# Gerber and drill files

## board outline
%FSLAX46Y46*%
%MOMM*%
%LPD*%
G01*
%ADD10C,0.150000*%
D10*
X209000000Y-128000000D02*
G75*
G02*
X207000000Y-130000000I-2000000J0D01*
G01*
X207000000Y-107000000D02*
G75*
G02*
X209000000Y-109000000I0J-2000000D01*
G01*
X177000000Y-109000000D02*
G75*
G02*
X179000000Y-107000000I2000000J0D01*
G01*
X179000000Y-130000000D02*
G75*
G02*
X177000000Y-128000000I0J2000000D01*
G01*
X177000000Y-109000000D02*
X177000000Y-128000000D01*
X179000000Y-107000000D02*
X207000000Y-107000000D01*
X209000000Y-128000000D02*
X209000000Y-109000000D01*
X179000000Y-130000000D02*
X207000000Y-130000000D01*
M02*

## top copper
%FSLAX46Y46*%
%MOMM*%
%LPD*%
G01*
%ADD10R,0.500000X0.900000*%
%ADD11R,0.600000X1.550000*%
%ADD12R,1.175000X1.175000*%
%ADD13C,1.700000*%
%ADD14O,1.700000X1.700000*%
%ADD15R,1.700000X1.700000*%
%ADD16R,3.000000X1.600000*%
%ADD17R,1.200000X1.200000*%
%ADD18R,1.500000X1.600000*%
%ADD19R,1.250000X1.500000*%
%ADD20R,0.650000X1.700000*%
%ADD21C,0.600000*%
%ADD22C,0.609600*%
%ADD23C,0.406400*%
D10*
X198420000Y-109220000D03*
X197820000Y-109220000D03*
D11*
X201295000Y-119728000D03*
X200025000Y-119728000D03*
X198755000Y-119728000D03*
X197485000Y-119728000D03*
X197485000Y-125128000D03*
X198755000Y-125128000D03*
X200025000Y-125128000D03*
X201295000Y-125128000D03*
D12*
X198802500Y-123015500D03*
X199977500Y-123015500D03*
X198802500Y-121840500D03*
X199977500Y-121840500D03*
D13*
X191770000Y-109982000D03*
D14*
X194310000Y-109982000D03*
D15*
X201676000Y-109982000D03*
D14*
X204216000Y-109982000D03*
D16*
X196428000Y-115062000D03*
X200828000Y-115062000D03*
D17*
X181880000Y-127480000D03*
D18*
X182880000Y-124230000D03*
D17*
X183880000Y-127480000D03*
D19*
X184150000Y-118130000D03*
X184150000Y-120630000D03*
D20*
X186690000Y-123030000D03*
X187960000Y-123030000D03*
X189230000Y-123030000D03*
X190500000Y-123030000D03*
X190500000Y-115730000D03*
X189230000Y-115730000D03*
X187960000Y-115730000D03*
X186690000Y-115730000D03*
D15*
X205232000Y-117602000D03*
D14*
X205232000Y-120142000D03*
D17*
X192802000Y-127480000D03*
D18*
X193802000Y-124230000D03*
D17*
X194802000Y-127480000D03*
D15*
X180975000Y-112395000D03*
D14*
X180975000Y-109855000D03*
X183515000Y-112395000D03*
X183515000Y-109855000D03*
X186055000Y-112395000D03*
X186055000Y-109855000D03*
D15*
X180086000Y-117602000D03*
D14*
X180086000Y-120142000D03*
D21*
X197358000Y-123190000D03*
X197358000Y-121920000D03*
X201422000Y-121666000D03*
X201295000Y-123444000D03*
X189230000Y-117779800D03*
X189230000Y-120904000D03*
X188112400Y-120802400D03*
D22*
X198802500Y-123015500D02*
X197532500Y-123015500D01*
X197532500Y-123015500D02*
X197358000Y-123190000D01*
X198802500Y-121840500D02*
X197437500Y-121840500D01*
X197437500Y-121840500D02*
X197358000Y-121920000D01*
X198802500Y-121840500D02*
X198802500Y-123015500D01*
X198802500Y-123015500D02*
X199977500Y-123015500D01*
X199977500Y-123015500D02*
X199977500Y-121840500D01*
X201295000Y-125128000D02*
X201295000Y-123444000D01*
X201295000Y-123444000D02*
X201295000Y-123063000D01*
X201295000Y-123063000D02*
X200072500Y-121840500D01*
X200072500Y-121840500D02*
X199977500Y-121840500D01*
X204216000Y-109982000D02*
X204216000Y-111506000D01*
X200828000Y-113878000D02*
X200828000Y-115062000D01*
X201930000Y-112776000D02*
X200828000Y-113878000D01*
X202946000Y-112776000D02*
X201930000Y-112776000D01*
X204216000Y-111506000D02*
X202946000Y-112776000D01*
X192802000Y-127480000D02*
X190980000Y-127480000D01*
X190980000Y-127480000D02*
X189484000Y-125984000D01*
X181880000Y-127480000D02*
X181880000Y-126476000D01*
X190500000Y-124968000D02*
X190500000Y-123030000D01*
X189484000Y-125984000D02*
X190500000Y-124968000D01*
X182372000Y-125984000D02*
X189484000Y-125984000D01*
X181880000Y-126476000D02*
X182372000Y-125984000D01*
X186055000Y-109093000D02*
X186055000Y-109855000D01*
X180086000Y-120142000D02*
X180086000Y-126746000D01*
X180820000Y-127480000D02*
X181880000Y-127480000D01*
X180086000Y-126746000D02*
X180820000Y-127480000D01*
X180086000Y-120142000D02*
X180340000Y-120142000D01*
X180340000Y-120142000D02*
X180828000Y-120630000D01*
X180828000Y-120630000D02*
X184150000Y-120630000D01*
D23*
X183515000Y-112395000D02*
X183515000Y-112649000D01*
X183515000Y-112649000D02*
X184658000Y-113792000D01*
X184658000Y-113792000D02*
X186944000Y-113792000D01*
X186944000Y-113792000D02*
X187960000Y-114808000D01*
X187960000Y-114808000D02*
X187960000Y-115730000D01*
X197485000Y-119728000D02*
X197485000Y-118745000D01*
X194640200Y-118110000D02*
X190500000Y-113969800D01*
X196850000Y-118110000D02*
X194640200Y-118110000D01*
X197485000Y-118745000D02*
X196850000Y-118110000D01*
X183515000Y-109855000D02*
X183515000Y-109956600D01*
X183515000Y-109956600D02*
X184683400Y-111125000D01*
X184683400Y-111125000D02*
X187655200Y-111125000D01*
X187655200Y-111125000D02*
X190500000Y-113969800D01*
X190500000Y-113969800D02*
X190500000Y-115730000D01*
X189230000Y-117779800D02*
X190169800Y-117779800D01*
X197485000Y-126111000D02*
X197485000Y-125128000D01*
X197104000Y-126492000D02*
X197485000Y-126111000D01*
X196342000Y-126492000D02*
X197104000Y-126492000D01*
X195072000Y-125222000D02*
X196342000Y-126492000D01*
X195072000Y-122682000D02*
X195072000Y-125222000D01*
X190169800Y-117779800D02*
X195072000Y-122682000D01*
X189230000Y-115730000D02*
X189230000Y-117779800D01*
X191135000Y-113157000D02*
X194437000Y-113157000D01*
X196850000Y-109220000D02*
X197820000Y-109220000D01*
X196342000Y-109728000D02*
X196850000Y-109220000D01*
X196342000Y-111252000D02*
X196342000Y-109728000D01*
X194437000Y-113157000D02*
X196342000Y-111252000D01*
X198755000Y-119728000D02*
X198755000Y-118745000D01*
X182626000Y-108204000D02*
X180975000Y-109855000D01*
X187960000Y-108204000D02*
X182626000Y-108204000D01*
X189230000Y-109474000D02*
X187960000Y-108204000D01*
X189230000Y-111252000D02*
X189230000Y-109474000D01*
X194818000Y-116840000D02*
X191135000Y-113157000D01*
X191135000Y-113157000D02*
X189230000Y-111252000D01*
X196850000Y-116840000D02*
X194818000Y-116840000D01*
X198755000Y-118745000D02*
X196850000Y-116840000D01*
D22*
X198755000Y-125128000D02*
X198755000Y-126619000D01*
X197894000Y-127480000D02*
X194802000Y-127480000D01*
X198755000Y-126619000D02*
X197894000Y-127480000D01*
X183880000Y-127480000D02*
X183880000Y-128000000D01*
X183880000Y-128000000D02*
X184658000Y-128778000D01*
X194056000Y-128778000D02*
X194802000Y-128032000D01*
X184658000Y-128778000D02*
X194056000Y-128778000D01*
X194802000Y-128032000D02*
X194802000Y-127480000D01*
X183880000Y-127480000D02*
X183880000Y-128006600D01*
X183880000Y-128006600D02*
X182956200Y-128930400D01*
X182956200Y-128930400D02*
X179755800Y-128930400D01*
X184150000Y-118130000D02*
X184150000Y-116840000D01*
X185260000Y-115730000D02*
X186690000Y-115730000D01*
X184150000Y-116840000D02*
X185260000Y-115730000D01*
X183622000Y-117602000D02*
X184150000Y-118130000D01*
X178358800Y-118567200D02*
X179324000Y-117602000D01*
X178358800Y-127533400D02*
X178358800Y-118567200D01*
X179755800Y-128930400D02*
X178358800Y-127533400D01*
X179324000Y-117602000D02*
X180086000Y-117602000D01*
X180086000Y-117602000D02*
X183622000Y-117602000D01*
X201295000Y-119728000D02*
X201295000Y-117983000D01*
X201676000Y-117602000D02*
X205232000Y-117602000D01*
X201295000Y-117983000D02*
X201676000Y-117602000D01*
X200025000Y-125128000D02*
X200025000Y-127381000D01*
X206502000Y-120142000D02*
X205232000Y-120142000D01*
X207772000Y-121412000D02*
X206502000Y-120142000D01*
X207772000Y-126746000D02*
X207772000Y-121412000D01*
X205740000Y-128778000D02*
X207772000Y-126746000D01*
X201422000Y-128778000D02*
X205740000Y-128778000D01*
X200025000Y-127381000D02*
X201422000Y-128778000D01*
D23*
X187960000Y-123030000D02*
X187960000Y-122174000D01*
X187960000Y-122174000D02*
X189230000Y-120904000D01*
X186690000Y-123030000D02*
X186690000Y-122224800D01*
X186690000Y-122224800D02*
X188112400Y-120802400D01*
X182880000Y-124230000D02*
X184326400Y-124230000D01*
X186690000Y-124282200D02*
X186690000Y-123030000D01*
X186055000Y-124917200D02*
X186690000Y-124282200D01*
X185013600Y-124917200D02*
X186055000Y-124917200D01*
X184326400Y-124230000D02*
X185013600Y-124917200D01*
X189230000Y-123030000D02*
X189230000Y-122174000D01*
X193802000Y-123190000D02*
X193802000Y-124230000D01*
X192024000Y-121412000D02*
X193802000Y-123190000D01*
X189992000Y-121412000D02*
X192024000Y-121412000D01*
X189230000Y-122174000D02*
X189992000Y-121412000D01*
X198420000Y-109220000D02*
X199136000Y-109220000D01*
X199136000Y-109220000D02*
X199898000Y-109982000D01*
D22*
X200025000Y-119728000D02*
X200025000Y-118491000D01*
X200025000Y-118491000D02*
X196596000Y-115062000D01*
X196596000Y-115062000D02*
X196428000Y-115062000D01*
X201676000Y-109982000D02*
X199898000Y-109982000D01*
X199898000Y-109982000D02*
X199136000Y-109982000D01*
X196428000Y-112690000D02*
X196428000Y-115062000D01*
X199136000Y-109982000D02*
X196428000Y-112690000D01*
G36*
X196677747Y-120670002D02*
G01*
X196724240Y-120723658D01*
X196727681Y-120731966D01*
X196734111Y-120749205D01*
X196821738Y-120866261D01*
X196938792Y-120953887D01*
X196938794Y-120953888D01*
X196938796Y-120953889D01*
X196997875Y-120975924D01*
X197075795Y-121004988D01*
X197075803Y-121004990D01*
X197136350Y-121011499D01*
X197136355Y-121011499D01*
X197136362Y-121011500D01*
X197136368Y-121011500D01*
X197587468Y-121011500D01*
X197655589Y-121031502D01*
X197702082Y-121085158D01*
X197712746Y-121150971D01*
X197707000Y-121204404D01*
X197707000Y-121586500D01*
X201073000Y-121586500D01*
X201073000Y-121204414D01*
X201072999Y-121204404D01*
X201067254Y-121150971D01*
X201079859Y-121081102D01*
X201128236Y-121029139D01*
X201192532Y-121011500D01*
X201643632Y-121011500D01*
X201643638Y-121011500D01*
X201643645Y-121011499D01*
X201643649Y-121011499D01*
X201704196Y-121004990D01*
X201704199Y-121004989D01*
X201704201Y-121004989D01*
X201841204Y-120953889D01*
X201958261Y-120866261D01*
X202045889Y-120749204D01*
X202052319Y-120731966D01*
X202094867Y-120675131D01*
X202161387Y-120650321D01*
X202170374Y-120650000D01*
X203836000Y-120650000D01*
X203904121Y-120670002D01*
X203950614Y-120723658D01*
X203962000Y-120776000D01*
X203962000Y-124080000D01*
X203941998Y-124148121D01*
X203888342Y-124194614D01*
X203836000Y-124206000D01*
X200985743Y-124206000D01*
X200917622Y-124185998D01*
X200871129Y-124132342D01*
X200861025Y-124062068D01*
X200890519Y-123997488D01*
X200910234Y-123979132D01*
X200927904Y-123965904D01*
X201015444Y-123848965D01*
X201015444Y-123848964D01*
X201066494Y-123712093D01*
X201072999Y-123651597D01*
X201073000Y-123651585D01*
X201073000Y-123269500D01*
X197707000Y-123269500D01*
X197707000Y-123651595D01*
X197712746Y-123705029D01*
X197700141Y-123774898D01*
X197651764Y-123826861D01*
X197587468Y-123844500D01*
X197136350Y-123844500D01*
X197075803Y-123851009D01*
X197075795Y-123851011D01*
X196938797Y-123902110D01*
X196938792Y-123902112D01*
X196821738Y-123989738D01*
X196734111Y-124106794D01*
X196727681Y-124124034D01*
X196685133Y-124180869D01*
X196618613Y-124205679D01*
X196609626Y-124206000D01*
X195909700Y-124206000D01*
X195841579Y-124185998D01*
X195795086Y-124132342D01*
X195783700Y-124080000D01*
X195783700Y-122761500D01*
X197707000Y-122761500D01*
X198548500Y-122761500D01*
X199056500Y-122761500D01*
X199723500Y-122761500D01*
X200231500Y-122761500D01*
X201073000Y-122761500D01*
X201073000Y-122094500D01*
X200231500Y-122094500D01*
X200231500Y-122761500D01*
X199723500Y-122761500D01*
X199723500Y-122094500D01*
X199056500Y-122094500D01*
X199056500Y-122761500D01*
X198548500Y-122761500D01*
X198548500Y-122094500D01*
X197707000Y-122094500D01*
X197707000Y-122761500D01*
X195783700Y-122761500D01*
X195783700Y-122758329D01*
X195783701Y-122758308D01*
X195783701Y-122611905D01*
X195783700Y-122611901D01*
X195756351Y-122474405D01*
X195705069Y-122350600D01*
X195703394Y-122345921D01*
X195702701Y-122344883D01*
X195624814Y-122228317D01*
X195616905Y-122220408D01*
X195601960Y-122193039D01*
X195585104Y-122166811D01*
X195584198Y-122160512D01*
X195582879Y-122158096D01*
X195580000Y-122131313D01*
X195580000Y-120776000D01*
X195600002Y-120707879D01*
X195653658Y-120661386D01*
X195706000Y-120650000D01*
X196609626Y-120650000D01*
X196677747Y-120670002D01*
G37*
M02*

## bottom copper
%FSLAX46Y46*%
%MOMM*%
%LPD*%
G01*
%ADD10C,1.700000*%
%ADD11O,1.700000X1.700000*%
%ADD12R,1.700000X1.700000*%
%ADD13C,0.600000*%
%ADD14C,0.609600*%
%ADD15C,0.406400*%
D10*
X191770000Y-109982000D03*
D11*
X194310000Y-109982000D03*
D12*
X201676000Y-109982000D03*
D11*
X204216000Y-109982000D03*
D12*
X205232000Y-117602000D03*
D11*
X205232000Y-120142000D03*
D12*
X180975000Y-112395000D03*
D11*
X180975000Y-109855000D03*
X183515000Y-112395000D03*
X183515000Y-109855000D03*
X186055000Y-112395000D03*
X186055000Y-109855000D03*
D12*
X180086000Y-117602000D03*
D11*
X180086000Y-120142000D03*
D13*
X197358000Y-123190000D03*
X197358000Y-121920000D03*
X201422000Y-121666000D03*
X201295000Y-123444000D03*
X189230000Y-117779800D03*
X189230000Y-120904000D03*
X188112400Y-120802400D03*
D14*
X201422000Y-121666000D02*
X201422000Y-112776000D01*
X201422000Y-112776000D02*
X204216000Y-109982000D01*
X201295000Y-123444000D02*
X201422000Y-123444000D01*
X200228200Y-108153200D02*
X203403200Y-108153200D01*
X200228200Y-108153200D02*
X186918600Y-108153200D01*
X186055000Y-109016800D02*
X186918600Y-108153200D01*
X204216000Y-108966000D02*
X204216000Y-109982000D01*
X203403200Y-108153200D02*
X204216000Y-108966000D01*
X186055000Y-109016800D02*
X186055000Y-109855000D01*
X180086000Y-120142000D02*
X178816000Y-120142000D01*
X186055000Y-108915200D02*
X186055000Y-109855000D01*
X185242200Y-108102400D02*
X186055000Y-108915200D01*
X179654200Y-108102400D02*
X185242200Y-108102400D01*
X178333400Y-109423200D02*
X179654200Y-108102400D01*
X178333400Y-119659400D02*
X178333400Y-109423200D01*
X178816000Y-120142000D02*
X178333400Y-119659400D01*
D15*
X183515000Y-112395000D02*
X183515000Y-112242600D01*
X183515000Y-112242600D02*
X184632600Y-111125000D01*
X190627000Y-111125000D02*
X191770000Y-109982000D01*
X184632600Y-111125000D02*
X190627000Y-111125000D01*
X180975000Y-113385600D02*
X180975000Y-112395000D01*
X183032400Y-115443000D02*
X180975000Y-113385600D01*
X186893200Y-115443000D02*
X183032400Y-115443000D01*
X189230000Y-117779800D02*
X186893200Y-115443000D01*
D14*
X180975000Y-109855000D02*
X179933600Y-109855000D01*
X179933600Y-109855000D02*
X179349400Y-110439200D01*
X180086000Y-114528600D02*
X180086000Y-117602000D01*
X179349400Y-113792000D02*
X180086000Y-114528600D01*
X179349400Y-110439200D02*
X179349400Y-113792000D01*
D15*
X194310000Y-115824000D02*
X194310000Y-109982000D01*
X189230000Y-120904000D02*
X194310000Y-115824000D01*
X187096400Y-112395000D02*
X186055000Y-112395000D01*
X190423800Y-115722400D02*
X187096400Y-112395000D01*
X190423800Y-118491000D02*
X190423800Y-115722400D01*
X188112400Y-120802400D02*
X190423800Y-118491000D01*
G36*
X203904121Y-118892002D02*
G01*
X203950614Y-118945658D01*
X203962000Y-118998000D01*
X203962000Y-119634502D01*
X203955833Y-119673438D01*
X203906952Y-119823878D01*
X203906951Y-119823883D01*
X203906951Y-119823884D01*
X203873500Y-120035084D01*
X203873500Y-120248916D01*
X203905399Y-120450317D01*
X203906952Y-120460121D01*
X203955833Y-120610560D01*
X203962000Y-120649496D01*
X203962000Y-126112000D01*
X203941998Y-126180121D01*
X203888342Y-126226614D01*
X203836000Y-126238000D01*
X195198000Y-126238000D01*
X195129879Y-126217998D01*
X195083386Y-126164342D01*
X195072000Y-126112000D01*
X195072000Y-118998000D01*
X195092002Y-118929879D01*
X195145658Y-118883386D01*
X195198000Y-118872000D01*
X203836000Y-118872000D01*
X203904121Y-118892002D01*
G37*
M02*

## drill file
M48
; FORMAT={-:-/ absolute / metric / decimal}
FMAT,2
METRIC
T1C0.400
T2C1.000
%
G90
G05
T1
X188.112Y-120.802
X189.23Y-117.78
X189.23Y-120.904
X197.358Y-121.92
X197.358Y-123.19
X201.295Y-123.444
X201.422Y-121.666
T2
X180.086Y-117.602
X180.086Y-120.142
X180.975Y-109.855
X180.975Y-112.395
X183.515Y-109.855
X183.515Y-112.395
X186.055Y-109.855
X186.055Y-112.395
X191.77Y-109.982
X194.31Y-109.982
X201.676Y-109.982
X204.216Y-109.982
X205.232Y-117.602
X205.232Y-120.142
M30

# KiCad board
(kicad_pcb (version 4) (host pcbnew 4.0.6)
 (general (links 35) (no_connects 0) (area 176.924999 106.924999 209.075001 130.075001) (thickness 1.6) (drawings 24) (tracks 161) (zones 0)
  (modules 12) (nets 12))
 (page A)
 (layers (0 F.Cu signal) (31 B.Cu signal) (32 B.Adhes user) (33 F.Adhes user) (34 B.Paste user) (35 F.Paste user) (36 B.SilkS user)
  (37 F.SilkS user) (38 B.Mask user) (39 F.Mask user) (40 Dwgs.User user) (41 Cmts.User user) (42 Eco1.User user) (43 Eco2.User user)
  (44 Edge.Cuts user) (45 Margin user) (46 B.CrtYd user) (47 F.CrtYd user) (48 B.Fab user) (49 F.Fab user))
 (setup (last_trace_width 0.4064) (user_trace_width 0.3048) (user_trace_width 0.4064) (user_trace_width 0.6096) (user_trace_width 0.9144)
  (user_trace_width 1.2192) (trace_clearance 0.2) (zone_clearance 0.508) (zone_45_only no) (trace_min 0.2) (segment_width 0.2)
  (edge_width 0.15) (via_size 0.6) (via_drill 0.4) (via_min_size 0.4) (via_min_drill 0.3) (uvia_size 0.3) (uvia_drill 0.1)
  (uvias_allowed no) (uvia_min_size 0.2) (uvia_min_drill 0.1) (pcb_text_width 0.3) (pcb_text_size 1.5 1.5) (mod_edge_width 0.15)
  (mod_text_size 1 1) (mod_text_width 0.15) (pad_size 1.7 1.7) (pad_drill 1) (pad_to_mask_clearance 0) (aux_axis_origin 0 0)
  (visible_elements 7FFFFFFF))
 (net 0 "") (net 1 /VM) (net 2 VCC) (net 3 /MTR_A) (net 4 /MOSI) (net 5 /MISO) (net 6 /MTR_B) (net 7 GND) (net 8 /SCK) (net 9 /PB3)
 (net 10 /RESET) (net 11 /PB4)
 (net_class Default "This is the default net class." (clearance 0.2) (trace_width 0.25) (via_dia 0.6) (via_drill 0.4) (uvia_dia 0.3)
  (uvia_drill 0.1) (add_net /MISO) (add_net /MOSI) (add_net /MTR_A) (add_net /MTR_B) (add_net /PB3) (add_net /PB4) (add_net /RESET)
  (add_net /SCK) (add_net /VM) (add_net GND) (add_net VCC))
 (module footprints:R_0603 (layer F.Cu) (at 198.12 109.22 180)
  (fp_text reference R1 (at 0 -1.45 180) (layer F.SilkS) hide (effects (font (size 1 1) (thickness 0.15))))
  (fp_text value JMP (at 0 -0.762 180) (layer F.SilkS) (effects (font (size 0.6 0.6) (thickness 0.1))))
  (pad 1 smd rect (at -0.3 0 180) (size 0.5 0.9) (layers F.Cu F.Paste F.Mask) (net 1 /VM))
  (pad 2 smd rect (at 0.3 0 180) (size 0.5 0.9) (layers F.Cu F.Paste F.Mask) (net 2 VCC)))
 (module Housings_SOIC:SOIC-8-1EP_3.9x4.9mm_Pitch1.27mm (layer F.Cu) (at 199.39 122.428 270)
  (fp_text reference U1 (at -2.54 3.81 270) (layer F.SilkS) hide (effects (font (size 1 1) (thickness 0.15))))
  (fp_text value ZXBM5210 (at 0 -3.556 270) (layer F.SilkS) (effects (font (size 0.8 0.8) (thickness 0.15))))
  (pad 1 smd rect (at -2.7 -1.905 270) (size 1.55 0.6) (layers F.Cu F.Paste F.Mask) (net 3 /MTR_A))
  (pad 2 smd rect (at -2.7 -0.635 270) (size 1.55 0.6) (layers F.Cu F.Paste F.Mask) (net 1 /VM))
  (pad 3 smd rect (at -2.7 0.635 270) (size 1.55 0.6) (layers F.Cu F.Paste F.Mask) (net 2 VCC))
  (pad 4 smd rect (at -2.7 1.905 270) (size 1.55 0.6) (layers F.Cu F.Paste F.Mask) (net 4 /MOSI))
  (pad 5 smd rect (at 2.7 1.905 270) (size 1.55 0.6) (layers F.Cu F.Paste F.Mask) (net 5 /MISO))
  (pad 6 smd rect (at 2.7 0.635 270) (size 1.55 0.6) (layers F.Cu F.Paste F.Mask) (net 2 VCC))
  (pad 7 smd rect (at 2.7 -0.635 270) (size 1.55 0.6) (layers F.Cu F.Paste F.Mask) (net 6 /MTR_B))
  (pad 8 smd rect (at 2.7 -1.905 270) (size 1.55 0.6) (layers F.Cu F.Paste F.Mask) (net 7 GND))
  (pad 8 smd rect (at 0.5875 0.5875 270) (size 1.175 1.175) (layers F.Cu F.Paste F.Mask) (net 7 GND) (solder_paste_margin_ratio -0.2))
  (pad 8 smd rect (at 0.5875 -0.5875 270) (size 1.175 1.175) (layers F.Cu F.Paste F.Mask) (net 7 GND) (solder_paste_margin_ratio -0.2))
  (pad 8 smd rect (at -0.5875 0.5875 270) (size 1.175 1.175) (layers F.Cu F.Paste F.Mask) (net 7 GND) (solder_paste_margin_ratio -0.2))
  (pad 8 smd rect (at -0.5875 -0.5875 270) (size 1.175 1.175) (layers F.Cu F.Paste F.Mask) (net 7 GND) (solder_paste_margin_ratio -0.2)))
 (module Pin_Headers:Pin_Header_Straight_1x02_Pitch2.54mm (layer F.Cu) (at 191.77 109.982 90)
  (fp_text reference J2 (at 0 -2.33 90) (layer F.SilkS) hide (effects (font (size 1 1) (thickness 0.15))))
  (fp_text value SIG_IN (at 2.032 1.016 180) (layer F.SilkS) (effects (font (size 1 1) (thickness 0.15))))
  (pad 1 thru_hole circle (at 0 0 90) (size 1.7 1.7) (drill 1) (layers *.Cu *.Mask) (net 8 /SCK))
  (pad 2 thru_hole oval (at 0 2.54 90) (size 1.7 1.7) (drill 1) (layers *.Cu *.Mask) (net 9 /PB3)))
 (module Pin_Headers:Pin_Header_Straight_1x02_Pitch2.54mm (layer F.Cu) (at 201.676 109.982 90)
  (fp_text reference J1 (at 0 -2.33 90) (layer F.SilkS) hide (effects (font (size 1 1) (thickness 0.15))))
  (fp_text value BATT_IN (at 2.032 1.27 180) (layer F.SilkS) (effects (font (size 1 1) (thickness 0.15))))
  (pad 1 thru_hole rect (at 0 0 90) (size 1.7 1.7) (drill 1) (layers *.Cu *.Mask) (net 1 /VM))
  (pad 2 thru_hole oval (at 0 2.54 90) (size 1.7 1.7) (drill 1) (layers *.Cu *.Mask) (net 7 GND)))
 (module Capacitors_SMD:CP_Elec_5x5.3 (layer F.Cu) (at 198.628 115.062)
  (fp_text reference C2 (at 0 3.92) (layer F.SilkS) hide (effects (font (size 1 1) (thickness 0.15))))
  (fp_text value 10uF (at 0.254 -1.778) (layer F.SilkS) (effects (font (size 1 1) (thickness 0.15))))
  (pad 1 smd rect (at -2.2 0 180) (size 3 1.6) (layers F.Cu F.Paste F.Mask) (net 1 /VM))
  (pad 2 smd rect (at 2.2 0 180) (size 3 1.6) (layers F.Cu F.Paste F.Mask) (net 7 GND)))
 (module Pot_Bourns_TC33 (layer F.Cu) (at 182.88 125.73)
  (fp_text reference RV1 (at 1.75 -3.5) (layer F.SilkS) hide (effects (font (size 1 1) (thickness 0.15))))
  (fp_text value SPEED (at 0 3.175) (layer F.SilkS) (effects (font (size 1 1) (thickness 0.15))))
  (pad 1 smd rect (at -1 1.75) (size 1.2 1.2) (layers F.Cu F.Mask) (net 7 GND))
  (pad 2 smd rect (at 0 -1.5) (size 1.5 1.6) (layers F.Cu F.Mask) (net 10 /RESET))
  (pad 3 smd rect (at 1 1.75) (size 1.2 1.2) (layers F.Cu F.Mask) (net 2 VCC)))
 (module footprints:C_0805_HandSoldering (layer F.Cu) (at 184.15 119.38 270)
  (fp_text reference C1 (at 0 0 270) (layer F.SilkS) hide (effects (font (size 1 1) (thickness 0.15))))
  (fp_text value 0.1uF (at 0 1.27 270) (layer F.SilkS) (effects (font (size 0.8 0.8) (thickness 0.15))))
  (pad 1 smd rect (at -1.25 0 270) (size 1.5 1.25) (layers F.Cu F.Paste F.Mask) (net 2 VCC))
  (pad 2 smd rect (at 1.25 0 270) (size 1.5 1.25) (layers F.Cu F.Paste F.Mask) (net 7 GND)))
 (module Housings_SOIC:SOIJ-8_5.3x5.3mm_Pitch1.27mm (layer F.Cu) (at 188.595 119.38 90)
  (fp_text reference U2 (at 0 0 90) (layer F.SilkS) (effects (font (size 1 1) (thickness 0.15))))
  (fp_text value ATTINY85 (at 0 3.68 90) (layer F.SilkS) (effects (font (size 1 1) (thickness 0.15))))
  (pad 1 smd rect (at -3.65 -1.905 90) (size 1.7 0.65) (layers F.Cu F.Paste F.Mask) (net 10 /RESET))
  (pad 2 smd rect (at -3.65 -0.635 90) (size 1.7 0.65) (layers F.Cu F.Paste F.Mask) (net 9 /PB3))
  (pad 3 smd rect (at -3.65 0.635 90) (size 1.7 0.65) (layers F.Cu F.Paste F.Mask) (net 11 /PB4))
  (pad 4 smd rect (at -3.65 1.905 90) (size 1.7 0.65) (layers F.Cu F.Paste F.Mask) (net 7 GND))
  (pad 5 smd rect (at 3.65 1.905 90) (size 1.7 0.65) (layers F.Cu F.Paste F.Mask) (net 4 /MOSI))
  (pad 6 smd rect (at 3.65 0.635 90) (size 1.7 0.65) (layers F.Cu F.Paste F.Mask) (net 5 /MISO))
  (pad 7 smd rect (at 3.65 -0.635 90) (size 1.7 0.65) (layers F.Cu F.Paste F.Mask) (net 8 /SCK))
  (pad 8 smd rect (at 3.65 -1.905 90) (size 1.7 0.65) (layers F.Cu F.Paste F.Mask) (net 2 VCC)))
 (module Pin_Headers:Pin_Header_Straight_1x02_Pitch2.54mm (layer F.Cu) (at 205.232 117.602)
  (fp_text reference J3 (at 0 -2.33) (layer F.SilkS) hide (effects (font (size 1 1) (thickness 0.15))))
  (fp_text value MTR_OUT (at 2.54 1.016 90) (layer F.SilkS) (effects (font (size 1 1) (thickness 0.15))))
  (pad 1 thru_hole rect (at 0 0) (size 1.7 1.7) (drill 1) (layers *.Cu *.Mask) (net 3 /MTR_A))
  (pad 2 thru_hole oval (at 0 2.54) (size 1.7 1.7) (drill 1) (layers *.Cu *.Mask) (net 6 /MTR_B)))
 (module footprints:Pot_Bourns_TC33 (layer F.Cu) (at 193.802 125.73)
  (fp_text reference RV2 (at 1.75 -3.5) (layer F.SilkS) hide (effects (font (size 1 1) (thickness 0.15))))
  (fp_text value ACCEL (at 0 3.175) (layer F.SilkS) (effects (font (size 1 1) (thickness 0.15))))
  (pad 1 smd rect (at -1 1.75) (size 1.2 1.2) (layers F.Cu F.Mask) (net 7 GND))
  (pad 2 smd rect (at 0 -1.5) (size 1.5 1.6) (layers F.Cu F.Mask) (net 11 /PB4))
  (pad 3 smd rect (at 1 1.75) (size 1.2 1.2) (layers F.Cu F.Mask) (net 2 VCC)))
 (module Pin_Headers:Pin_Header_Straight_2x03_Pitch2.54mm (layer F.Cu) (at 180.975 112.395 90)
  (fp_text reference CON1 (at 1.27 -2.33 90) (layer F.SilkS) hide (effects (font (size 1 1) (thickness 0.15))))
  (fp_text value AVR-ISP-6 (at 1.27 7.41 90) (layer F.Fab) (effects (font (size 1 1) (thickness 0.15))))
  (pad 1 thru_hole rect (at 0 0 90) (size 1.7 1.7) (drill 1) (layers *.Cu *.Mask) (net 5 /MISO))
  (pad 2 thru_hole oval (at 2.54 0 90) (size 1.7 1.7) (drill 1) (layers *.Cu *.Mask) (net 2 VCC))
  (pad 3 thru_hole oval (at 0 2.54 90) (size 1.7 1.7) (drill 1) (layers *.Cu *.Mask) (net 8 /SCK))
  (pad 4 thru_hole oval (at 2.54 2.54 90) (size 1.7 1.7) (drill 1) (layers *.Cu *.Mask) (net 4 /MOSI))
  (pad 5 thru_hole oval (at 0 5.08 90) (size 1.7 1.7) (drill 1) (layers *.Cu *.Mask) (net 10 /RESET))
  (pad 6 thru_hole oval (at 2.54 5.08 90) (size 1.7 1.7) (drill 1) (layers *.Cu *.Mask) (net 7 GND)))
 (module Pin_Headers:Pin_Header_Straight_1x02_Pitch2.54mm (layer F.Cu) (at 180.086 117.602)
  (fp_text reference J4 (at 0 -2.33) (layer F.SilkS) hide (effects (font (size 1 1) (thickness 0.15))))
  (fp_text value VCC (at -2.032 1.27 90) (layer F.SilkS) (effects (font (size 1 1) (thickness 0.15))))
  (pad 1 thru_hole rect (at 0 0) (size 1.7 1.7) (drill 1) (layers *.Cu *.Mask) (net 2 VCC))
  (pad 2 thru_hole oval (at 0 2.54) (size 1.7 1.7) (drill 1) (layers *.Cu *.Mask) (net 7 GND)))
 (gr_arc (start 207 128) (end 209 128) (angle 90) (layer Edge.Cuts) (width 0.15))
 (gr_arc (start 207 109) (end 207 107) (angle 90) (layer Edge.Cuts) (width 0.15))
 (gr_arc (start 179 109) (end 177 109) (angle 90) (layer Edge.Cuts) (width 0.15))
 (gr_arc (start 179 128) (end 179 130) (angle 90) (layer Edge.Cuts) (width 0.15))
 (gr_line (start 177 109) (end 177 128) (angle 90) (layer Edge.Cuts) (width 0.15))
 (gr_line (start 179 107) (end 207 107) (angle 90) (layer Edge.Cuts) (width 0.15))
 (gr_line (start 209 128) (end 209 109) (angle 90) (layer Edge.Cuts) (width 0.15))
 (gr_line (start 179 130) (end 207 130) (angle 90) (layer Edge.Cuts) (width 0.15))
 (segment (start 198.8025 123.0155) (end 197.5325 123.0155) (width 0.6096) (layer F.Cu) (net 7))
 (via (at 197.358 123.19) (size 0.6) (drill 0.4) (layers F.Cu B.Cu) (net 7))
 (segment (start 197.5325 123.0155) (end 197.358 123.19) (width 0.6096) (layer F.Cu) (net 7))
 (segment (start 198.8025 121.8405) (end 197.4375 121.8405) (width 0.6096) (layer F.Cu) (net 7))
 (via (at 197.358 121.92) (size 0.6) (drill 0.4) (layers F.Cu B.Cu) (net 7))
 (segment (start 197.4375 121.8405) (end 197.358 121.92) (width 0.6096) (layer F.Cu) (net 7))
 (segment (start 201.422 121.666) (end 201.422 112.776) (width 0.6096) (layer B.Cu) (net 7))
 (via (at 201.422 121.666) (size 0.6) (drill 0.4) (layers F.Cu B.Cu) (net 7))
 (segment (start 201.422 112.776) (end 204.216 109.982) (width 0.6096) (layer B.Cu) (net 7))
 (via (at 201.295 123.444) (size 0.6) (drill 0.4) (layers F.Cu B.Cu) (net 7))
 (segment (start 201.295 123.444) (end 201.422 123.444) (width 0.6096) (layer B.Cu) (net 7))
 (segment (start 198.8025 121.8405) (end 198.8025 123.0155) (width 0.6096) (layer F.Cu) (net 7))
 (segment (start 198.8025 123.0155) (end 199.9775 123.0155) (width 0.6096) (layer F.Cu) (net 7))
 (segment (start 199.9775 123.0155) (end 199.9775 121.8405) (width 0.6096) (layer F.Cu) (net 7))
 (segment (start 201.295 125.128) (end 201.295 123.444) (width 0.6096) (layer F.Cu) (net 7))
 (segment (start 201.295 123.444) (end 201.295 123.063) (width 0.6096) (layer F.Cu) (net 7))
 (segment (start 201.295 123.063) (end 200.0725 121.8405) (width 0.6096) (layer F.Cu) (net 7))
 (segment (start 200.0725 121.8405) (end 199.9775 121.8405) (width 0.6096) (layer F.Cu) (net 7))
 (segment (start 204.216 109.982) (end 204.216 111.506) (width 0.6096) (layer F.Cu) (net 7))
 (segment (start 200.828 113.878) (end 200.828 115.062) (width 0.6096) (layer F.Cu) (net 7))
 (segment (start 201.93 112.776) (end 200.828 113.878) (width 0.6096) (layer F.Cu) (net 7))
 (segment (start 202.946 112.776) (end 201.93 112.776) (width 0.6096) (layer F.Cu) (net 7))
 (segment (start 204.216 111.506) (end 202.946 112.776) (width 0.6096) (layer F.Cu) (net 7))
 (segment (start 192.802 127.48) (end 190.98 127.48) (width 0.6096) (layer F.Cu) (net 7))
 (segment (start 190.98 127.48) (end 189.484 125.984) (width 0.6096) (layer F.Cu) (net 7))
 (segment (start 200.2282 108.1532) (end 203.4032 108.1532) (width 0.6096) (layer B.Cu) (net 7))
 (segment (start 200.2282 108.1532) (end 186.9186 108.1532) (width 0.6096) (layer B.Cu) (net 7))
 (segment (start 186.055 109.0168) (end 186.9186 108.1532) (width 0.6096) (layer B.Cu) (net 7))
 (segment (start 204.216 108.966) (end 204.216 109.982) (width 0.6096) (layer B.Cu) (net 7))
 (segment (start 203.4032 108.1532) (end 204.216 108.966) (width 0.6096) (layer B.Cu) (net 7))
 (segment (start 186.055 109.0168) (end 186.055 109.855) (width 0.6096) (layer B.Cu) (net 7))
 (segment (start 180.086 120.142) (end 178.816 120.142) (width 0.6096) (layer B.Cu) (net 7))
 (segment (start 186.055 108.9152) (end 186.055 109.855) (width 0.6096) (layer B.Cu) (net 7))
 (segment (start 185.2422 108.1024) (end 186.055 108.9152) (width 0.6096) (layer B.Cu) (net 7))
 (segment (start 179.6542 108.1024) (end 185.2422 108.1024) (width 0.6096) (layer B.Cu) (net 7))
 (segment (start 178.3334 109.4232) (end 179.6542 108.1024) (width 0.6096) (layer B.Cu) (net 7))
 (segment (start 178.3334 119.6594) (end 178.3334 109.4232) (width 0.6096) (layer B.Cu) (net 7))
 (segment (start 178.816 120.142) (end 178.3334 119.6594) (width 0.6096) (layer B.Cu) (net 7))
 (segment (start 181.88 127.48) (end 181.88 126.476) (width 0.6096) (layer F.Cu) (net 7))
 (segment (start 190.5 124.968) (end 190.5 123.03) (width 0.6096) (layer F.Cu) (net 7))
 (segment (start 189.484 125.984) (end 190.5 124.968) (width 0.6096) (layer F.Cu) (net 7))
 (segment (start 182.372 125.984) (end 189.484 125.984) (width 0.6096) (layer F.Cu) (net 7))
 (segment (start 181.88 126.476) (end 182.372 125.984) (width 0.6096) (layer F.Cu) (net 7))
 (segment (start 186.055 109.093) (end 186.055 109.855) (width 0.6096) (layer F.Cu) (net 7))
 (segment (start 180.086 120.142) (end 180.086 126.746) (width 0.6096) (layer F.Cu) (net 7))
 (segment (start 180.82 127.48) (end 181.88 127.48) (width 0.6096) (layer F.Cu) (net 7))
 (segment (start 180.086 126.746) (end 180.82 127.48) (width 0.6096) (layer F.Cu) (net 7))
 (segment (start 180.086 120.142) (end 180.34 120.142) (width 0.6096) (layer F.Cu) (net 7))
 (segment (start 180.34 120.142) (end 180.828 120.63) (width 0.6096) (layer F.Cu) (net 7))
 (segment (start 180.828 120.63) (end 184.15 120.63) (width 0.6096) (layer F.Cu) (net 7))
 (segment (start 183.515 112.395) (end 183.515 112.2426) (width 0.4064) (layer B.Cu) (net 8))
 (segment (start 183.515 112.2426) (end 184.6326 111.125) (width 0.4064) (layer B.Cu) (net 8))
 (segment (start 190.627 111.125) (end 191.77 109.982) (width 0.4064) (layer B.Cu) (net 8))
 (segment (start 184.6326 111.125) (end 190.627 111.125) (width 0.4064) (layer B.Cu) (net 8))
 (segment (start 183.515 112.395) (end 183.515 112.649) (width 0.4064) (layer F.Cu) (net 8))
 (segment (start 183.515 112.649) (end 184.658 113.792) (width 0.4064) (layer F.Cu) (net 8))
 (segment (start 184.658 113.792) (end 186.944 113.792) (width 0.4064) (layer F.Cu) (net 8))
 (segment (start 186.944 113.792) (end 187.96 114.808) (width 0.4064) (layer F.Cu) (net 8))
 (segment (start 187.96 114.808) (end 187.96 115.73) (width 0.4064) (layer F.Cu) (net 8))
 (segment (start 197.485 119.728) (end 197.485 118.745) (width 0.4064) (layer F.Cu) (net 4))
 (segment (start 194.6402 118.11) (end 190.5 113.9698) (width 0.4064) (layer F.Cu) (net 4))
 (segment (start 196.85 118.11) (end 194.6402 118.11) (width 0.4064) (layer F.Cu) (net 4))
 (segment (start 197.485 118.745) (end 196.85 118.11) (width 0.4064) (layer F.Cu) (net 4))
 (segment (start 183.515 109.855) (end 183.515 109.9566) (width 0.4064) (layer F.Cu) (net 4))
 (segment (start 183.515 109.9566) (end 184.6834 111.125) (width 0.4064) (layer F.Cu) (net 4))
 (segment (start 184.6834 111.125) (end 187.6552 111.125) (width 0.4064) (layer F.Cu) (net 4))
 (segment (start 187.6552 111.125) (end 190.5 113.9698) (width 0.4064) (layer F.Cu) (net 4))
 (segment (start 190.5 113.9698) (end 190.5 115.73) (width 0.4064) (layer F.Cu) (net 4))
 (segment (start 189.23 117.7798) (end 190.1698 117.7798) (width 0.4064) (layer F.Cu) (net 5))
 (segment (start 197.485 126.111) (end 197.485 125.128) (width 0.4064) (layer F.Cu) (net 5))
 (segment (start 197.104 126.492) (end 197.485 126.111) (width 0.4064) (layer F.Cu) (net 5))
 (segment (start 196.342 126.492) (end 197.104 126.492) (width 0.4064) (layer F.Cu) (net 5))
 (segment (start 195.072 125.222) (end 196.342 126.492) (width 0.4064) (layer F.Cu) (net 5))
 (segment (start 195.072 122.682) (end 195.072 125.222) (width 0.4064) (layer F.Cu) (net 5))
 (segment (start 190.1698 117.7798) (end 195.072 122.682) (width 0.4064) (layer F.Cu) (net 5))
 (segment (start 189.23 115.73) (end 189.23 117.7798) (width 0.4064) (layer F.Cu) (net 5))
 (via (at 189.23 117.7798) (size 0.6) (drill 0.4) (layers F.Cu B.Cu) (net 5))
 (segment (start 180.975 113.3856) (end 180.975 112.395) (width 0.4064) (layer B.Cu) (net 5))
 (segment (start 183.0324 115.443) (end 180.975 113.3856) (width 0.4064) (layer B.Cu) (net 5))
 (segment (start 186.8932 115.443) (end 183.0324 115.443) (width 0.4064) (layer B.Cu) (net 5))
 (segment (start 189.23 117.7798) (end 186.8932 115.443) (width 0.4064) (layer B.Cu) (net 5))
 (segment (start 191.135 113.157) (end 194.437 113.157) (width 0.4064) (layer F.Cu) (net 2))
 (segment (start 196.85 109.22) (end 197.82 109.22) (width 0.4064) (layer F.Cu) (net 2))
 (segment (start 196.342 109.728) (end 196.85 109.22) (width 0.4064) (layer F.Cu) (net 2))
 (segment (start 196.342 111.252) (end 196.342 109.728) (width 0.4064) (layer F.Cu) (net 2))
 (segment (start 194.437 113.157) (end 196.342 111.252) (width 0.4064) (layer F.Cu) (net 2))
 (segment (start 198.755 119.728) (end 198.755 118.745) (width 0.4064) (layer F.Cu) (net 2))
 (segment (start 182.626 108.204) (end 180.975 109.855) (width 0.4064) (layer F.Cu) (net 2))
 (segment (start 187.96 108.204) (end 182.626 108.204) (width 0.4064) (layer F.Cu) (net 2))
 (segment (start 189.23 109.474) (end 187.96 108.204) (width 0.4064) (layer F.Cu) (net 2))
 (segment (start 189.23 111.252) (end 189.23 109.474) (width 0.4064) (layer F.Cu) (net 2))
 (segment (start 194.818 116.84) (end 191.135 113.157) (width 0.4064) (layer F.Cu) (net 2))
 (segment (start 191.135 113.157) (end 189.23 111.252) (width 0.4064) (layer F.Cu) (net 2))
 (segment (start 196.85 116.84) (end 194.818 116.84) (width 0.4064) (layer F.Cu) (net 2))
 (segment (start 198.755 118.745) (end 196.85 116.84) (width 0.4064) (layer F.Cu) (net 2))
 (segment (start 198.755 125.128) (end 198.755 126.619) (width 0.6096) (layer F.Cu) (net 2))
 (segment (start 197.894 127.48) (end 194.802 127.48) (width 0.6096) (layer F.Cu) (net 2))
 (segment (start 198.755 126.619) (end 197.894 127.48) (width 0.6096) (layer F.Cu) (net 2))
 (segment (start 183.88 127.48) (end 183.88 128) (width 0.6096) (layer F.Cu) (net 2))
 (segment (start 183.88 128) (end 184.658 128.778) (width 0.6096) (layer F.Cu) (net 2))
 (segment (start 194.056 128.778) (end 194.802 128.032) (width 0.6096) (layer F.Cu) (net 2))
 (segment (start 184.658 128.778) (end 194.056 128.778) (width 0.6096) (layer F.Cu) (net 2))
 (segment (start 194.802 128.032) (end 194.802 127.48) (width 0.6096) (layer F.Cu) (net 2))
 (segment (start 183.88 127.48) (end 183.88 128.0066) (width 0.6096) (layer F.Cu) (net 2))
 (segment (start 183.88 128.0066) (end 182.9562 128.9304) (width 0.6096) (layer F.Cu) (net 2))
 (segment (start 182.9562 128.9304) (end 179.7558 128.9304) (width 0.6096) (layer F.Cu) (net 2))
 (segment (start 180.975 109.855) (end 179.9336 109.855) (width 0.6096) (layer B.Cu) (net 2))
 (segment (start 179.9336 109.855) (end 179.3494 110.4392) (width 0.6096) (layer B.Cu) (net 2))
 (segment (start 184.15 118.13) (end 184.15 116.84) (width 0.6096) (layer F.Cu) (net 2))
 (segment (start 185.26 115.73) (end 186.69 115.73) (width 0.6096) (layer F.Cu) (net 2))
 (segment (start 184.15 116.84) (end 185.26 115.73) (width 0.6096) (layer F.Cu) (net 2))
 (segment (start 183.622 117.602) (end 184.15 118.13) (width 0.6096) (layer F.Cu) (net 2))
 (segment (start 178.3588 118.5672) (end 179.324 117.602) (width 0.6096) (layer F.Cu) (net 2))
 (segment (start 178.3588 127.5334) (end 178.3588 118.5672) (width 0.6096) (layer F.Cu) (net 2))
 (segment (start 179.7558 128.9304) (end 178.3588 127.5334) (width 0.6096) (layer F.Cu) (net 2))
 (segment (start 179.324 117.602) (end 180.086 117.602) (width 0.6096) (layer F.Cu) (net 2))
 (segment (start 180.086 114.5286) (end 180.086 117.602) (width 0.6096) (layer B.Cu) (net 2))
 (segment (start 179.3494 113.792) (end 180.086 114.5286) (width 0.6096) (layer B.Cu) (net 2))
 (segment (start 179.3494 110.4392) (end 179.3494 113.792) (width 0.6096) (layer B.Cu) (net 2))
 (segment (start 180.086 117.602) (end 183.622 117.602) (width 0.6096) (layer F.Cu) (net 2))
 (segment (start 201.295 119.728) (end 201.295 117.983) (width 0.6096) (layer F.Cu) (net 3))
 (segment (start 201.676 117.602) (end 205.232 117.602) (width 0.6096) (layer F.Cu) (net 3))
 (segment (start 201.295 117.983) (end 201.676 117.602) (width 0.6096) (layer F.Cu) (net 3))
 (segment (start 200.025 125.128) (end 200.025 127.381) (width 0.6096) (layer F.Cu) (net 6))
 (segment (start 206.502 120.142) (end 205.232 120.142) (width 0.6096) (layer F.Cu) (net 6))
 (segment (start 207.772 121.412) (end 206.502 120.142) (width 0.6096) (layer F.Cu) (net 6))
 (segment (start 207.772 126.746) (end 207.772 121.412) (width 0.6096) (layer F.Cu) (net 6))
 (segment (start 205.74 128.778) (end 207.772 126.746) (width 0.6096) (layer F.Cu) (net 6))
 (segment (start 201.422 128.778) (end 205.74 128.778) (width 0.6096) (layer F.Cu) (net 6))
 (segment (start 200.025 127.381) (end 201.422 128.778) (width 0.6096) (layer F.Cu) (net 6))
 (segment (start 187.96 123.03) (end 187.96 122.174) (width 0.4064) (layer F.Cu) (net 9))
 (segment (start 194.31 115.824) (end 194.31 109.982) (width 0.4064) (layer B.Cu) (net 9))
 (segment (start 189.23 120.904) (end 194.31 115.824) (width 0.4064) (layer B.Cu) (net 9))
 (via (at 189.23 120.904) (size 0.6) (drill 0.4) (layers F.Cu B.Cu) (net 9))
 (segment (start 187.96 122.174) (end 189.23 120.904) (width 0.4064) (layer F.Cu) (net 9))
 (segment (start 186.69 123.03) (end 186.69 122.2248) (width 0.4064) (layer F.Cu) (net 10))
 (segment (start 186.69 122.2248) (end 188.1124 120.8024) (width 0.4064) (layer F.Cu) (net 10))
 (segment (start 187.0964 112.395) (end 186.055 112.395) (width 0.4064) (layer B.Cu) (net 10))
 (segment (start 190.4238 115.7224) (end 187.0964 112.395) (width 0.4064) (layer B.Cu) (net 10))
 (segment (start 190.4238 118.491) (end 190.4238 115.7224) (width 0.4064) (layer B.Cu) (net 10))
 (segment (start 188.1124 120.8024) (end 190.4238 118.491) (width 0.4064) (layer B.Cu) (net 10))
 (via (at 188.1124 120.8024) (size 0.6) (drill 0.4) (layers F.Cu B.Cu) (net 10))
 (segment (start 182.88 124.23) (end 184.3264 124.23) (width 0.4064) (layer F.Cu) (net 10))
 (segment (start 186.69 124.2822) (end 186.69 123.03) (width 0.4064) (layer F.Cu) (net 10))
 (segment (start 186.055 124.9172) (end 186.69 124.2822) (width 0.4064) (layer F.Cu) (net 10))
 (segment (start 185.0136 124.9172) (end 186.055 124.9172) (width 0.4064) (layer F.Cu) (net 10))
 (segment (start 184.3264 124.23) (end 185.0136 124.9172) (width 0.4064) (layer F.Cu) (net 10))
 (segment (start 189.23 123.03) (end 189.23 122.174) (width 0.4064) (layer F.Cu) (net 11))
 (segment (start 193.802 123.19) (end 193.802 124.23) (width 0.4064) (layer F.Cu) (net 11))
 (segment (start 192.024 121.412) (end 193.802 123.19) (width 0.4064) (layer F.Cu) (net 11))
 (segment (start 189.992 121.412) (end 192.024 121.412) (width 0.4064) (layer F.Cu) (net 11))
 (segment (start 189.23 122.174) (end 189.992 121.412) (width 0.4064) (layer F.Cu) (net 11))
 (segment (start 198.42 109.22) (end 199.136 109.22) (width 0.4064) (layer F.Cu) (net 1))
 (segment (start 199.136 109.22) (end 199.898 109.982) (width 0.4064) (layer F.Cu) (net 1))
 (segment (start 200.025 119.728) (end 200.025 118.491) (width 0.6096) (layer F.Cu) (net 1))
 (segment (start 200.025 118.491) (end 196.596 115.062) (width 0.6096) (layer F.Cu) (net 1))
 (segment (start 196.596 115.062) (end 196.428 115.062) (width 0.6096) (layer F.Cu) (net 1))
 (segment (start 201.676 109.982) (end 199.898 109.982) (width 0.6096) (layer F.Cu) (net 1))
 (segment (start 199.898 109.982) (end 199.136 109.982) (width 0.6096) (layer F.Cu) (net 1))
 (segment (start 196.428 112.69) (end 196.428 115.062) (width 0.6096) (layer F.Cu) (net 1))
 (segment (start 199.136 109.982) (end 196.428 112.69) (width 0.6096) (layer F.Cu) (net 1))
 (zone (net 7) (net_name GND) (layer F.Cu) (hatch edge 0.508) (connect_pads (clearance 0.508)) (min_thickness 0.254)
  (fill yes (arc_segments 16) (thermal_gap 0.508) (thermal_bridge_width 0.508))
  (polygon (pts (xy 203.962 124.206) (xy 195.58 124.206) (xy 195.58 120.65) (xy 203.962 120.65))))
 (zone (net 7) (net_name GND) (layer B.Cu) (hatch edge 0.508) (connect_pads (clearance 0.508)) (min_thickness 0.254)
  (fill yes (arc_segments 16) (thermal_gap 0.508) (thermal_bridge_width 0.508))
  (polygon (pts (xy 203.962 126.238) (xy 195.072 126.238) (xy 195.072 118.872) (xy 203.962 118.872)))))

